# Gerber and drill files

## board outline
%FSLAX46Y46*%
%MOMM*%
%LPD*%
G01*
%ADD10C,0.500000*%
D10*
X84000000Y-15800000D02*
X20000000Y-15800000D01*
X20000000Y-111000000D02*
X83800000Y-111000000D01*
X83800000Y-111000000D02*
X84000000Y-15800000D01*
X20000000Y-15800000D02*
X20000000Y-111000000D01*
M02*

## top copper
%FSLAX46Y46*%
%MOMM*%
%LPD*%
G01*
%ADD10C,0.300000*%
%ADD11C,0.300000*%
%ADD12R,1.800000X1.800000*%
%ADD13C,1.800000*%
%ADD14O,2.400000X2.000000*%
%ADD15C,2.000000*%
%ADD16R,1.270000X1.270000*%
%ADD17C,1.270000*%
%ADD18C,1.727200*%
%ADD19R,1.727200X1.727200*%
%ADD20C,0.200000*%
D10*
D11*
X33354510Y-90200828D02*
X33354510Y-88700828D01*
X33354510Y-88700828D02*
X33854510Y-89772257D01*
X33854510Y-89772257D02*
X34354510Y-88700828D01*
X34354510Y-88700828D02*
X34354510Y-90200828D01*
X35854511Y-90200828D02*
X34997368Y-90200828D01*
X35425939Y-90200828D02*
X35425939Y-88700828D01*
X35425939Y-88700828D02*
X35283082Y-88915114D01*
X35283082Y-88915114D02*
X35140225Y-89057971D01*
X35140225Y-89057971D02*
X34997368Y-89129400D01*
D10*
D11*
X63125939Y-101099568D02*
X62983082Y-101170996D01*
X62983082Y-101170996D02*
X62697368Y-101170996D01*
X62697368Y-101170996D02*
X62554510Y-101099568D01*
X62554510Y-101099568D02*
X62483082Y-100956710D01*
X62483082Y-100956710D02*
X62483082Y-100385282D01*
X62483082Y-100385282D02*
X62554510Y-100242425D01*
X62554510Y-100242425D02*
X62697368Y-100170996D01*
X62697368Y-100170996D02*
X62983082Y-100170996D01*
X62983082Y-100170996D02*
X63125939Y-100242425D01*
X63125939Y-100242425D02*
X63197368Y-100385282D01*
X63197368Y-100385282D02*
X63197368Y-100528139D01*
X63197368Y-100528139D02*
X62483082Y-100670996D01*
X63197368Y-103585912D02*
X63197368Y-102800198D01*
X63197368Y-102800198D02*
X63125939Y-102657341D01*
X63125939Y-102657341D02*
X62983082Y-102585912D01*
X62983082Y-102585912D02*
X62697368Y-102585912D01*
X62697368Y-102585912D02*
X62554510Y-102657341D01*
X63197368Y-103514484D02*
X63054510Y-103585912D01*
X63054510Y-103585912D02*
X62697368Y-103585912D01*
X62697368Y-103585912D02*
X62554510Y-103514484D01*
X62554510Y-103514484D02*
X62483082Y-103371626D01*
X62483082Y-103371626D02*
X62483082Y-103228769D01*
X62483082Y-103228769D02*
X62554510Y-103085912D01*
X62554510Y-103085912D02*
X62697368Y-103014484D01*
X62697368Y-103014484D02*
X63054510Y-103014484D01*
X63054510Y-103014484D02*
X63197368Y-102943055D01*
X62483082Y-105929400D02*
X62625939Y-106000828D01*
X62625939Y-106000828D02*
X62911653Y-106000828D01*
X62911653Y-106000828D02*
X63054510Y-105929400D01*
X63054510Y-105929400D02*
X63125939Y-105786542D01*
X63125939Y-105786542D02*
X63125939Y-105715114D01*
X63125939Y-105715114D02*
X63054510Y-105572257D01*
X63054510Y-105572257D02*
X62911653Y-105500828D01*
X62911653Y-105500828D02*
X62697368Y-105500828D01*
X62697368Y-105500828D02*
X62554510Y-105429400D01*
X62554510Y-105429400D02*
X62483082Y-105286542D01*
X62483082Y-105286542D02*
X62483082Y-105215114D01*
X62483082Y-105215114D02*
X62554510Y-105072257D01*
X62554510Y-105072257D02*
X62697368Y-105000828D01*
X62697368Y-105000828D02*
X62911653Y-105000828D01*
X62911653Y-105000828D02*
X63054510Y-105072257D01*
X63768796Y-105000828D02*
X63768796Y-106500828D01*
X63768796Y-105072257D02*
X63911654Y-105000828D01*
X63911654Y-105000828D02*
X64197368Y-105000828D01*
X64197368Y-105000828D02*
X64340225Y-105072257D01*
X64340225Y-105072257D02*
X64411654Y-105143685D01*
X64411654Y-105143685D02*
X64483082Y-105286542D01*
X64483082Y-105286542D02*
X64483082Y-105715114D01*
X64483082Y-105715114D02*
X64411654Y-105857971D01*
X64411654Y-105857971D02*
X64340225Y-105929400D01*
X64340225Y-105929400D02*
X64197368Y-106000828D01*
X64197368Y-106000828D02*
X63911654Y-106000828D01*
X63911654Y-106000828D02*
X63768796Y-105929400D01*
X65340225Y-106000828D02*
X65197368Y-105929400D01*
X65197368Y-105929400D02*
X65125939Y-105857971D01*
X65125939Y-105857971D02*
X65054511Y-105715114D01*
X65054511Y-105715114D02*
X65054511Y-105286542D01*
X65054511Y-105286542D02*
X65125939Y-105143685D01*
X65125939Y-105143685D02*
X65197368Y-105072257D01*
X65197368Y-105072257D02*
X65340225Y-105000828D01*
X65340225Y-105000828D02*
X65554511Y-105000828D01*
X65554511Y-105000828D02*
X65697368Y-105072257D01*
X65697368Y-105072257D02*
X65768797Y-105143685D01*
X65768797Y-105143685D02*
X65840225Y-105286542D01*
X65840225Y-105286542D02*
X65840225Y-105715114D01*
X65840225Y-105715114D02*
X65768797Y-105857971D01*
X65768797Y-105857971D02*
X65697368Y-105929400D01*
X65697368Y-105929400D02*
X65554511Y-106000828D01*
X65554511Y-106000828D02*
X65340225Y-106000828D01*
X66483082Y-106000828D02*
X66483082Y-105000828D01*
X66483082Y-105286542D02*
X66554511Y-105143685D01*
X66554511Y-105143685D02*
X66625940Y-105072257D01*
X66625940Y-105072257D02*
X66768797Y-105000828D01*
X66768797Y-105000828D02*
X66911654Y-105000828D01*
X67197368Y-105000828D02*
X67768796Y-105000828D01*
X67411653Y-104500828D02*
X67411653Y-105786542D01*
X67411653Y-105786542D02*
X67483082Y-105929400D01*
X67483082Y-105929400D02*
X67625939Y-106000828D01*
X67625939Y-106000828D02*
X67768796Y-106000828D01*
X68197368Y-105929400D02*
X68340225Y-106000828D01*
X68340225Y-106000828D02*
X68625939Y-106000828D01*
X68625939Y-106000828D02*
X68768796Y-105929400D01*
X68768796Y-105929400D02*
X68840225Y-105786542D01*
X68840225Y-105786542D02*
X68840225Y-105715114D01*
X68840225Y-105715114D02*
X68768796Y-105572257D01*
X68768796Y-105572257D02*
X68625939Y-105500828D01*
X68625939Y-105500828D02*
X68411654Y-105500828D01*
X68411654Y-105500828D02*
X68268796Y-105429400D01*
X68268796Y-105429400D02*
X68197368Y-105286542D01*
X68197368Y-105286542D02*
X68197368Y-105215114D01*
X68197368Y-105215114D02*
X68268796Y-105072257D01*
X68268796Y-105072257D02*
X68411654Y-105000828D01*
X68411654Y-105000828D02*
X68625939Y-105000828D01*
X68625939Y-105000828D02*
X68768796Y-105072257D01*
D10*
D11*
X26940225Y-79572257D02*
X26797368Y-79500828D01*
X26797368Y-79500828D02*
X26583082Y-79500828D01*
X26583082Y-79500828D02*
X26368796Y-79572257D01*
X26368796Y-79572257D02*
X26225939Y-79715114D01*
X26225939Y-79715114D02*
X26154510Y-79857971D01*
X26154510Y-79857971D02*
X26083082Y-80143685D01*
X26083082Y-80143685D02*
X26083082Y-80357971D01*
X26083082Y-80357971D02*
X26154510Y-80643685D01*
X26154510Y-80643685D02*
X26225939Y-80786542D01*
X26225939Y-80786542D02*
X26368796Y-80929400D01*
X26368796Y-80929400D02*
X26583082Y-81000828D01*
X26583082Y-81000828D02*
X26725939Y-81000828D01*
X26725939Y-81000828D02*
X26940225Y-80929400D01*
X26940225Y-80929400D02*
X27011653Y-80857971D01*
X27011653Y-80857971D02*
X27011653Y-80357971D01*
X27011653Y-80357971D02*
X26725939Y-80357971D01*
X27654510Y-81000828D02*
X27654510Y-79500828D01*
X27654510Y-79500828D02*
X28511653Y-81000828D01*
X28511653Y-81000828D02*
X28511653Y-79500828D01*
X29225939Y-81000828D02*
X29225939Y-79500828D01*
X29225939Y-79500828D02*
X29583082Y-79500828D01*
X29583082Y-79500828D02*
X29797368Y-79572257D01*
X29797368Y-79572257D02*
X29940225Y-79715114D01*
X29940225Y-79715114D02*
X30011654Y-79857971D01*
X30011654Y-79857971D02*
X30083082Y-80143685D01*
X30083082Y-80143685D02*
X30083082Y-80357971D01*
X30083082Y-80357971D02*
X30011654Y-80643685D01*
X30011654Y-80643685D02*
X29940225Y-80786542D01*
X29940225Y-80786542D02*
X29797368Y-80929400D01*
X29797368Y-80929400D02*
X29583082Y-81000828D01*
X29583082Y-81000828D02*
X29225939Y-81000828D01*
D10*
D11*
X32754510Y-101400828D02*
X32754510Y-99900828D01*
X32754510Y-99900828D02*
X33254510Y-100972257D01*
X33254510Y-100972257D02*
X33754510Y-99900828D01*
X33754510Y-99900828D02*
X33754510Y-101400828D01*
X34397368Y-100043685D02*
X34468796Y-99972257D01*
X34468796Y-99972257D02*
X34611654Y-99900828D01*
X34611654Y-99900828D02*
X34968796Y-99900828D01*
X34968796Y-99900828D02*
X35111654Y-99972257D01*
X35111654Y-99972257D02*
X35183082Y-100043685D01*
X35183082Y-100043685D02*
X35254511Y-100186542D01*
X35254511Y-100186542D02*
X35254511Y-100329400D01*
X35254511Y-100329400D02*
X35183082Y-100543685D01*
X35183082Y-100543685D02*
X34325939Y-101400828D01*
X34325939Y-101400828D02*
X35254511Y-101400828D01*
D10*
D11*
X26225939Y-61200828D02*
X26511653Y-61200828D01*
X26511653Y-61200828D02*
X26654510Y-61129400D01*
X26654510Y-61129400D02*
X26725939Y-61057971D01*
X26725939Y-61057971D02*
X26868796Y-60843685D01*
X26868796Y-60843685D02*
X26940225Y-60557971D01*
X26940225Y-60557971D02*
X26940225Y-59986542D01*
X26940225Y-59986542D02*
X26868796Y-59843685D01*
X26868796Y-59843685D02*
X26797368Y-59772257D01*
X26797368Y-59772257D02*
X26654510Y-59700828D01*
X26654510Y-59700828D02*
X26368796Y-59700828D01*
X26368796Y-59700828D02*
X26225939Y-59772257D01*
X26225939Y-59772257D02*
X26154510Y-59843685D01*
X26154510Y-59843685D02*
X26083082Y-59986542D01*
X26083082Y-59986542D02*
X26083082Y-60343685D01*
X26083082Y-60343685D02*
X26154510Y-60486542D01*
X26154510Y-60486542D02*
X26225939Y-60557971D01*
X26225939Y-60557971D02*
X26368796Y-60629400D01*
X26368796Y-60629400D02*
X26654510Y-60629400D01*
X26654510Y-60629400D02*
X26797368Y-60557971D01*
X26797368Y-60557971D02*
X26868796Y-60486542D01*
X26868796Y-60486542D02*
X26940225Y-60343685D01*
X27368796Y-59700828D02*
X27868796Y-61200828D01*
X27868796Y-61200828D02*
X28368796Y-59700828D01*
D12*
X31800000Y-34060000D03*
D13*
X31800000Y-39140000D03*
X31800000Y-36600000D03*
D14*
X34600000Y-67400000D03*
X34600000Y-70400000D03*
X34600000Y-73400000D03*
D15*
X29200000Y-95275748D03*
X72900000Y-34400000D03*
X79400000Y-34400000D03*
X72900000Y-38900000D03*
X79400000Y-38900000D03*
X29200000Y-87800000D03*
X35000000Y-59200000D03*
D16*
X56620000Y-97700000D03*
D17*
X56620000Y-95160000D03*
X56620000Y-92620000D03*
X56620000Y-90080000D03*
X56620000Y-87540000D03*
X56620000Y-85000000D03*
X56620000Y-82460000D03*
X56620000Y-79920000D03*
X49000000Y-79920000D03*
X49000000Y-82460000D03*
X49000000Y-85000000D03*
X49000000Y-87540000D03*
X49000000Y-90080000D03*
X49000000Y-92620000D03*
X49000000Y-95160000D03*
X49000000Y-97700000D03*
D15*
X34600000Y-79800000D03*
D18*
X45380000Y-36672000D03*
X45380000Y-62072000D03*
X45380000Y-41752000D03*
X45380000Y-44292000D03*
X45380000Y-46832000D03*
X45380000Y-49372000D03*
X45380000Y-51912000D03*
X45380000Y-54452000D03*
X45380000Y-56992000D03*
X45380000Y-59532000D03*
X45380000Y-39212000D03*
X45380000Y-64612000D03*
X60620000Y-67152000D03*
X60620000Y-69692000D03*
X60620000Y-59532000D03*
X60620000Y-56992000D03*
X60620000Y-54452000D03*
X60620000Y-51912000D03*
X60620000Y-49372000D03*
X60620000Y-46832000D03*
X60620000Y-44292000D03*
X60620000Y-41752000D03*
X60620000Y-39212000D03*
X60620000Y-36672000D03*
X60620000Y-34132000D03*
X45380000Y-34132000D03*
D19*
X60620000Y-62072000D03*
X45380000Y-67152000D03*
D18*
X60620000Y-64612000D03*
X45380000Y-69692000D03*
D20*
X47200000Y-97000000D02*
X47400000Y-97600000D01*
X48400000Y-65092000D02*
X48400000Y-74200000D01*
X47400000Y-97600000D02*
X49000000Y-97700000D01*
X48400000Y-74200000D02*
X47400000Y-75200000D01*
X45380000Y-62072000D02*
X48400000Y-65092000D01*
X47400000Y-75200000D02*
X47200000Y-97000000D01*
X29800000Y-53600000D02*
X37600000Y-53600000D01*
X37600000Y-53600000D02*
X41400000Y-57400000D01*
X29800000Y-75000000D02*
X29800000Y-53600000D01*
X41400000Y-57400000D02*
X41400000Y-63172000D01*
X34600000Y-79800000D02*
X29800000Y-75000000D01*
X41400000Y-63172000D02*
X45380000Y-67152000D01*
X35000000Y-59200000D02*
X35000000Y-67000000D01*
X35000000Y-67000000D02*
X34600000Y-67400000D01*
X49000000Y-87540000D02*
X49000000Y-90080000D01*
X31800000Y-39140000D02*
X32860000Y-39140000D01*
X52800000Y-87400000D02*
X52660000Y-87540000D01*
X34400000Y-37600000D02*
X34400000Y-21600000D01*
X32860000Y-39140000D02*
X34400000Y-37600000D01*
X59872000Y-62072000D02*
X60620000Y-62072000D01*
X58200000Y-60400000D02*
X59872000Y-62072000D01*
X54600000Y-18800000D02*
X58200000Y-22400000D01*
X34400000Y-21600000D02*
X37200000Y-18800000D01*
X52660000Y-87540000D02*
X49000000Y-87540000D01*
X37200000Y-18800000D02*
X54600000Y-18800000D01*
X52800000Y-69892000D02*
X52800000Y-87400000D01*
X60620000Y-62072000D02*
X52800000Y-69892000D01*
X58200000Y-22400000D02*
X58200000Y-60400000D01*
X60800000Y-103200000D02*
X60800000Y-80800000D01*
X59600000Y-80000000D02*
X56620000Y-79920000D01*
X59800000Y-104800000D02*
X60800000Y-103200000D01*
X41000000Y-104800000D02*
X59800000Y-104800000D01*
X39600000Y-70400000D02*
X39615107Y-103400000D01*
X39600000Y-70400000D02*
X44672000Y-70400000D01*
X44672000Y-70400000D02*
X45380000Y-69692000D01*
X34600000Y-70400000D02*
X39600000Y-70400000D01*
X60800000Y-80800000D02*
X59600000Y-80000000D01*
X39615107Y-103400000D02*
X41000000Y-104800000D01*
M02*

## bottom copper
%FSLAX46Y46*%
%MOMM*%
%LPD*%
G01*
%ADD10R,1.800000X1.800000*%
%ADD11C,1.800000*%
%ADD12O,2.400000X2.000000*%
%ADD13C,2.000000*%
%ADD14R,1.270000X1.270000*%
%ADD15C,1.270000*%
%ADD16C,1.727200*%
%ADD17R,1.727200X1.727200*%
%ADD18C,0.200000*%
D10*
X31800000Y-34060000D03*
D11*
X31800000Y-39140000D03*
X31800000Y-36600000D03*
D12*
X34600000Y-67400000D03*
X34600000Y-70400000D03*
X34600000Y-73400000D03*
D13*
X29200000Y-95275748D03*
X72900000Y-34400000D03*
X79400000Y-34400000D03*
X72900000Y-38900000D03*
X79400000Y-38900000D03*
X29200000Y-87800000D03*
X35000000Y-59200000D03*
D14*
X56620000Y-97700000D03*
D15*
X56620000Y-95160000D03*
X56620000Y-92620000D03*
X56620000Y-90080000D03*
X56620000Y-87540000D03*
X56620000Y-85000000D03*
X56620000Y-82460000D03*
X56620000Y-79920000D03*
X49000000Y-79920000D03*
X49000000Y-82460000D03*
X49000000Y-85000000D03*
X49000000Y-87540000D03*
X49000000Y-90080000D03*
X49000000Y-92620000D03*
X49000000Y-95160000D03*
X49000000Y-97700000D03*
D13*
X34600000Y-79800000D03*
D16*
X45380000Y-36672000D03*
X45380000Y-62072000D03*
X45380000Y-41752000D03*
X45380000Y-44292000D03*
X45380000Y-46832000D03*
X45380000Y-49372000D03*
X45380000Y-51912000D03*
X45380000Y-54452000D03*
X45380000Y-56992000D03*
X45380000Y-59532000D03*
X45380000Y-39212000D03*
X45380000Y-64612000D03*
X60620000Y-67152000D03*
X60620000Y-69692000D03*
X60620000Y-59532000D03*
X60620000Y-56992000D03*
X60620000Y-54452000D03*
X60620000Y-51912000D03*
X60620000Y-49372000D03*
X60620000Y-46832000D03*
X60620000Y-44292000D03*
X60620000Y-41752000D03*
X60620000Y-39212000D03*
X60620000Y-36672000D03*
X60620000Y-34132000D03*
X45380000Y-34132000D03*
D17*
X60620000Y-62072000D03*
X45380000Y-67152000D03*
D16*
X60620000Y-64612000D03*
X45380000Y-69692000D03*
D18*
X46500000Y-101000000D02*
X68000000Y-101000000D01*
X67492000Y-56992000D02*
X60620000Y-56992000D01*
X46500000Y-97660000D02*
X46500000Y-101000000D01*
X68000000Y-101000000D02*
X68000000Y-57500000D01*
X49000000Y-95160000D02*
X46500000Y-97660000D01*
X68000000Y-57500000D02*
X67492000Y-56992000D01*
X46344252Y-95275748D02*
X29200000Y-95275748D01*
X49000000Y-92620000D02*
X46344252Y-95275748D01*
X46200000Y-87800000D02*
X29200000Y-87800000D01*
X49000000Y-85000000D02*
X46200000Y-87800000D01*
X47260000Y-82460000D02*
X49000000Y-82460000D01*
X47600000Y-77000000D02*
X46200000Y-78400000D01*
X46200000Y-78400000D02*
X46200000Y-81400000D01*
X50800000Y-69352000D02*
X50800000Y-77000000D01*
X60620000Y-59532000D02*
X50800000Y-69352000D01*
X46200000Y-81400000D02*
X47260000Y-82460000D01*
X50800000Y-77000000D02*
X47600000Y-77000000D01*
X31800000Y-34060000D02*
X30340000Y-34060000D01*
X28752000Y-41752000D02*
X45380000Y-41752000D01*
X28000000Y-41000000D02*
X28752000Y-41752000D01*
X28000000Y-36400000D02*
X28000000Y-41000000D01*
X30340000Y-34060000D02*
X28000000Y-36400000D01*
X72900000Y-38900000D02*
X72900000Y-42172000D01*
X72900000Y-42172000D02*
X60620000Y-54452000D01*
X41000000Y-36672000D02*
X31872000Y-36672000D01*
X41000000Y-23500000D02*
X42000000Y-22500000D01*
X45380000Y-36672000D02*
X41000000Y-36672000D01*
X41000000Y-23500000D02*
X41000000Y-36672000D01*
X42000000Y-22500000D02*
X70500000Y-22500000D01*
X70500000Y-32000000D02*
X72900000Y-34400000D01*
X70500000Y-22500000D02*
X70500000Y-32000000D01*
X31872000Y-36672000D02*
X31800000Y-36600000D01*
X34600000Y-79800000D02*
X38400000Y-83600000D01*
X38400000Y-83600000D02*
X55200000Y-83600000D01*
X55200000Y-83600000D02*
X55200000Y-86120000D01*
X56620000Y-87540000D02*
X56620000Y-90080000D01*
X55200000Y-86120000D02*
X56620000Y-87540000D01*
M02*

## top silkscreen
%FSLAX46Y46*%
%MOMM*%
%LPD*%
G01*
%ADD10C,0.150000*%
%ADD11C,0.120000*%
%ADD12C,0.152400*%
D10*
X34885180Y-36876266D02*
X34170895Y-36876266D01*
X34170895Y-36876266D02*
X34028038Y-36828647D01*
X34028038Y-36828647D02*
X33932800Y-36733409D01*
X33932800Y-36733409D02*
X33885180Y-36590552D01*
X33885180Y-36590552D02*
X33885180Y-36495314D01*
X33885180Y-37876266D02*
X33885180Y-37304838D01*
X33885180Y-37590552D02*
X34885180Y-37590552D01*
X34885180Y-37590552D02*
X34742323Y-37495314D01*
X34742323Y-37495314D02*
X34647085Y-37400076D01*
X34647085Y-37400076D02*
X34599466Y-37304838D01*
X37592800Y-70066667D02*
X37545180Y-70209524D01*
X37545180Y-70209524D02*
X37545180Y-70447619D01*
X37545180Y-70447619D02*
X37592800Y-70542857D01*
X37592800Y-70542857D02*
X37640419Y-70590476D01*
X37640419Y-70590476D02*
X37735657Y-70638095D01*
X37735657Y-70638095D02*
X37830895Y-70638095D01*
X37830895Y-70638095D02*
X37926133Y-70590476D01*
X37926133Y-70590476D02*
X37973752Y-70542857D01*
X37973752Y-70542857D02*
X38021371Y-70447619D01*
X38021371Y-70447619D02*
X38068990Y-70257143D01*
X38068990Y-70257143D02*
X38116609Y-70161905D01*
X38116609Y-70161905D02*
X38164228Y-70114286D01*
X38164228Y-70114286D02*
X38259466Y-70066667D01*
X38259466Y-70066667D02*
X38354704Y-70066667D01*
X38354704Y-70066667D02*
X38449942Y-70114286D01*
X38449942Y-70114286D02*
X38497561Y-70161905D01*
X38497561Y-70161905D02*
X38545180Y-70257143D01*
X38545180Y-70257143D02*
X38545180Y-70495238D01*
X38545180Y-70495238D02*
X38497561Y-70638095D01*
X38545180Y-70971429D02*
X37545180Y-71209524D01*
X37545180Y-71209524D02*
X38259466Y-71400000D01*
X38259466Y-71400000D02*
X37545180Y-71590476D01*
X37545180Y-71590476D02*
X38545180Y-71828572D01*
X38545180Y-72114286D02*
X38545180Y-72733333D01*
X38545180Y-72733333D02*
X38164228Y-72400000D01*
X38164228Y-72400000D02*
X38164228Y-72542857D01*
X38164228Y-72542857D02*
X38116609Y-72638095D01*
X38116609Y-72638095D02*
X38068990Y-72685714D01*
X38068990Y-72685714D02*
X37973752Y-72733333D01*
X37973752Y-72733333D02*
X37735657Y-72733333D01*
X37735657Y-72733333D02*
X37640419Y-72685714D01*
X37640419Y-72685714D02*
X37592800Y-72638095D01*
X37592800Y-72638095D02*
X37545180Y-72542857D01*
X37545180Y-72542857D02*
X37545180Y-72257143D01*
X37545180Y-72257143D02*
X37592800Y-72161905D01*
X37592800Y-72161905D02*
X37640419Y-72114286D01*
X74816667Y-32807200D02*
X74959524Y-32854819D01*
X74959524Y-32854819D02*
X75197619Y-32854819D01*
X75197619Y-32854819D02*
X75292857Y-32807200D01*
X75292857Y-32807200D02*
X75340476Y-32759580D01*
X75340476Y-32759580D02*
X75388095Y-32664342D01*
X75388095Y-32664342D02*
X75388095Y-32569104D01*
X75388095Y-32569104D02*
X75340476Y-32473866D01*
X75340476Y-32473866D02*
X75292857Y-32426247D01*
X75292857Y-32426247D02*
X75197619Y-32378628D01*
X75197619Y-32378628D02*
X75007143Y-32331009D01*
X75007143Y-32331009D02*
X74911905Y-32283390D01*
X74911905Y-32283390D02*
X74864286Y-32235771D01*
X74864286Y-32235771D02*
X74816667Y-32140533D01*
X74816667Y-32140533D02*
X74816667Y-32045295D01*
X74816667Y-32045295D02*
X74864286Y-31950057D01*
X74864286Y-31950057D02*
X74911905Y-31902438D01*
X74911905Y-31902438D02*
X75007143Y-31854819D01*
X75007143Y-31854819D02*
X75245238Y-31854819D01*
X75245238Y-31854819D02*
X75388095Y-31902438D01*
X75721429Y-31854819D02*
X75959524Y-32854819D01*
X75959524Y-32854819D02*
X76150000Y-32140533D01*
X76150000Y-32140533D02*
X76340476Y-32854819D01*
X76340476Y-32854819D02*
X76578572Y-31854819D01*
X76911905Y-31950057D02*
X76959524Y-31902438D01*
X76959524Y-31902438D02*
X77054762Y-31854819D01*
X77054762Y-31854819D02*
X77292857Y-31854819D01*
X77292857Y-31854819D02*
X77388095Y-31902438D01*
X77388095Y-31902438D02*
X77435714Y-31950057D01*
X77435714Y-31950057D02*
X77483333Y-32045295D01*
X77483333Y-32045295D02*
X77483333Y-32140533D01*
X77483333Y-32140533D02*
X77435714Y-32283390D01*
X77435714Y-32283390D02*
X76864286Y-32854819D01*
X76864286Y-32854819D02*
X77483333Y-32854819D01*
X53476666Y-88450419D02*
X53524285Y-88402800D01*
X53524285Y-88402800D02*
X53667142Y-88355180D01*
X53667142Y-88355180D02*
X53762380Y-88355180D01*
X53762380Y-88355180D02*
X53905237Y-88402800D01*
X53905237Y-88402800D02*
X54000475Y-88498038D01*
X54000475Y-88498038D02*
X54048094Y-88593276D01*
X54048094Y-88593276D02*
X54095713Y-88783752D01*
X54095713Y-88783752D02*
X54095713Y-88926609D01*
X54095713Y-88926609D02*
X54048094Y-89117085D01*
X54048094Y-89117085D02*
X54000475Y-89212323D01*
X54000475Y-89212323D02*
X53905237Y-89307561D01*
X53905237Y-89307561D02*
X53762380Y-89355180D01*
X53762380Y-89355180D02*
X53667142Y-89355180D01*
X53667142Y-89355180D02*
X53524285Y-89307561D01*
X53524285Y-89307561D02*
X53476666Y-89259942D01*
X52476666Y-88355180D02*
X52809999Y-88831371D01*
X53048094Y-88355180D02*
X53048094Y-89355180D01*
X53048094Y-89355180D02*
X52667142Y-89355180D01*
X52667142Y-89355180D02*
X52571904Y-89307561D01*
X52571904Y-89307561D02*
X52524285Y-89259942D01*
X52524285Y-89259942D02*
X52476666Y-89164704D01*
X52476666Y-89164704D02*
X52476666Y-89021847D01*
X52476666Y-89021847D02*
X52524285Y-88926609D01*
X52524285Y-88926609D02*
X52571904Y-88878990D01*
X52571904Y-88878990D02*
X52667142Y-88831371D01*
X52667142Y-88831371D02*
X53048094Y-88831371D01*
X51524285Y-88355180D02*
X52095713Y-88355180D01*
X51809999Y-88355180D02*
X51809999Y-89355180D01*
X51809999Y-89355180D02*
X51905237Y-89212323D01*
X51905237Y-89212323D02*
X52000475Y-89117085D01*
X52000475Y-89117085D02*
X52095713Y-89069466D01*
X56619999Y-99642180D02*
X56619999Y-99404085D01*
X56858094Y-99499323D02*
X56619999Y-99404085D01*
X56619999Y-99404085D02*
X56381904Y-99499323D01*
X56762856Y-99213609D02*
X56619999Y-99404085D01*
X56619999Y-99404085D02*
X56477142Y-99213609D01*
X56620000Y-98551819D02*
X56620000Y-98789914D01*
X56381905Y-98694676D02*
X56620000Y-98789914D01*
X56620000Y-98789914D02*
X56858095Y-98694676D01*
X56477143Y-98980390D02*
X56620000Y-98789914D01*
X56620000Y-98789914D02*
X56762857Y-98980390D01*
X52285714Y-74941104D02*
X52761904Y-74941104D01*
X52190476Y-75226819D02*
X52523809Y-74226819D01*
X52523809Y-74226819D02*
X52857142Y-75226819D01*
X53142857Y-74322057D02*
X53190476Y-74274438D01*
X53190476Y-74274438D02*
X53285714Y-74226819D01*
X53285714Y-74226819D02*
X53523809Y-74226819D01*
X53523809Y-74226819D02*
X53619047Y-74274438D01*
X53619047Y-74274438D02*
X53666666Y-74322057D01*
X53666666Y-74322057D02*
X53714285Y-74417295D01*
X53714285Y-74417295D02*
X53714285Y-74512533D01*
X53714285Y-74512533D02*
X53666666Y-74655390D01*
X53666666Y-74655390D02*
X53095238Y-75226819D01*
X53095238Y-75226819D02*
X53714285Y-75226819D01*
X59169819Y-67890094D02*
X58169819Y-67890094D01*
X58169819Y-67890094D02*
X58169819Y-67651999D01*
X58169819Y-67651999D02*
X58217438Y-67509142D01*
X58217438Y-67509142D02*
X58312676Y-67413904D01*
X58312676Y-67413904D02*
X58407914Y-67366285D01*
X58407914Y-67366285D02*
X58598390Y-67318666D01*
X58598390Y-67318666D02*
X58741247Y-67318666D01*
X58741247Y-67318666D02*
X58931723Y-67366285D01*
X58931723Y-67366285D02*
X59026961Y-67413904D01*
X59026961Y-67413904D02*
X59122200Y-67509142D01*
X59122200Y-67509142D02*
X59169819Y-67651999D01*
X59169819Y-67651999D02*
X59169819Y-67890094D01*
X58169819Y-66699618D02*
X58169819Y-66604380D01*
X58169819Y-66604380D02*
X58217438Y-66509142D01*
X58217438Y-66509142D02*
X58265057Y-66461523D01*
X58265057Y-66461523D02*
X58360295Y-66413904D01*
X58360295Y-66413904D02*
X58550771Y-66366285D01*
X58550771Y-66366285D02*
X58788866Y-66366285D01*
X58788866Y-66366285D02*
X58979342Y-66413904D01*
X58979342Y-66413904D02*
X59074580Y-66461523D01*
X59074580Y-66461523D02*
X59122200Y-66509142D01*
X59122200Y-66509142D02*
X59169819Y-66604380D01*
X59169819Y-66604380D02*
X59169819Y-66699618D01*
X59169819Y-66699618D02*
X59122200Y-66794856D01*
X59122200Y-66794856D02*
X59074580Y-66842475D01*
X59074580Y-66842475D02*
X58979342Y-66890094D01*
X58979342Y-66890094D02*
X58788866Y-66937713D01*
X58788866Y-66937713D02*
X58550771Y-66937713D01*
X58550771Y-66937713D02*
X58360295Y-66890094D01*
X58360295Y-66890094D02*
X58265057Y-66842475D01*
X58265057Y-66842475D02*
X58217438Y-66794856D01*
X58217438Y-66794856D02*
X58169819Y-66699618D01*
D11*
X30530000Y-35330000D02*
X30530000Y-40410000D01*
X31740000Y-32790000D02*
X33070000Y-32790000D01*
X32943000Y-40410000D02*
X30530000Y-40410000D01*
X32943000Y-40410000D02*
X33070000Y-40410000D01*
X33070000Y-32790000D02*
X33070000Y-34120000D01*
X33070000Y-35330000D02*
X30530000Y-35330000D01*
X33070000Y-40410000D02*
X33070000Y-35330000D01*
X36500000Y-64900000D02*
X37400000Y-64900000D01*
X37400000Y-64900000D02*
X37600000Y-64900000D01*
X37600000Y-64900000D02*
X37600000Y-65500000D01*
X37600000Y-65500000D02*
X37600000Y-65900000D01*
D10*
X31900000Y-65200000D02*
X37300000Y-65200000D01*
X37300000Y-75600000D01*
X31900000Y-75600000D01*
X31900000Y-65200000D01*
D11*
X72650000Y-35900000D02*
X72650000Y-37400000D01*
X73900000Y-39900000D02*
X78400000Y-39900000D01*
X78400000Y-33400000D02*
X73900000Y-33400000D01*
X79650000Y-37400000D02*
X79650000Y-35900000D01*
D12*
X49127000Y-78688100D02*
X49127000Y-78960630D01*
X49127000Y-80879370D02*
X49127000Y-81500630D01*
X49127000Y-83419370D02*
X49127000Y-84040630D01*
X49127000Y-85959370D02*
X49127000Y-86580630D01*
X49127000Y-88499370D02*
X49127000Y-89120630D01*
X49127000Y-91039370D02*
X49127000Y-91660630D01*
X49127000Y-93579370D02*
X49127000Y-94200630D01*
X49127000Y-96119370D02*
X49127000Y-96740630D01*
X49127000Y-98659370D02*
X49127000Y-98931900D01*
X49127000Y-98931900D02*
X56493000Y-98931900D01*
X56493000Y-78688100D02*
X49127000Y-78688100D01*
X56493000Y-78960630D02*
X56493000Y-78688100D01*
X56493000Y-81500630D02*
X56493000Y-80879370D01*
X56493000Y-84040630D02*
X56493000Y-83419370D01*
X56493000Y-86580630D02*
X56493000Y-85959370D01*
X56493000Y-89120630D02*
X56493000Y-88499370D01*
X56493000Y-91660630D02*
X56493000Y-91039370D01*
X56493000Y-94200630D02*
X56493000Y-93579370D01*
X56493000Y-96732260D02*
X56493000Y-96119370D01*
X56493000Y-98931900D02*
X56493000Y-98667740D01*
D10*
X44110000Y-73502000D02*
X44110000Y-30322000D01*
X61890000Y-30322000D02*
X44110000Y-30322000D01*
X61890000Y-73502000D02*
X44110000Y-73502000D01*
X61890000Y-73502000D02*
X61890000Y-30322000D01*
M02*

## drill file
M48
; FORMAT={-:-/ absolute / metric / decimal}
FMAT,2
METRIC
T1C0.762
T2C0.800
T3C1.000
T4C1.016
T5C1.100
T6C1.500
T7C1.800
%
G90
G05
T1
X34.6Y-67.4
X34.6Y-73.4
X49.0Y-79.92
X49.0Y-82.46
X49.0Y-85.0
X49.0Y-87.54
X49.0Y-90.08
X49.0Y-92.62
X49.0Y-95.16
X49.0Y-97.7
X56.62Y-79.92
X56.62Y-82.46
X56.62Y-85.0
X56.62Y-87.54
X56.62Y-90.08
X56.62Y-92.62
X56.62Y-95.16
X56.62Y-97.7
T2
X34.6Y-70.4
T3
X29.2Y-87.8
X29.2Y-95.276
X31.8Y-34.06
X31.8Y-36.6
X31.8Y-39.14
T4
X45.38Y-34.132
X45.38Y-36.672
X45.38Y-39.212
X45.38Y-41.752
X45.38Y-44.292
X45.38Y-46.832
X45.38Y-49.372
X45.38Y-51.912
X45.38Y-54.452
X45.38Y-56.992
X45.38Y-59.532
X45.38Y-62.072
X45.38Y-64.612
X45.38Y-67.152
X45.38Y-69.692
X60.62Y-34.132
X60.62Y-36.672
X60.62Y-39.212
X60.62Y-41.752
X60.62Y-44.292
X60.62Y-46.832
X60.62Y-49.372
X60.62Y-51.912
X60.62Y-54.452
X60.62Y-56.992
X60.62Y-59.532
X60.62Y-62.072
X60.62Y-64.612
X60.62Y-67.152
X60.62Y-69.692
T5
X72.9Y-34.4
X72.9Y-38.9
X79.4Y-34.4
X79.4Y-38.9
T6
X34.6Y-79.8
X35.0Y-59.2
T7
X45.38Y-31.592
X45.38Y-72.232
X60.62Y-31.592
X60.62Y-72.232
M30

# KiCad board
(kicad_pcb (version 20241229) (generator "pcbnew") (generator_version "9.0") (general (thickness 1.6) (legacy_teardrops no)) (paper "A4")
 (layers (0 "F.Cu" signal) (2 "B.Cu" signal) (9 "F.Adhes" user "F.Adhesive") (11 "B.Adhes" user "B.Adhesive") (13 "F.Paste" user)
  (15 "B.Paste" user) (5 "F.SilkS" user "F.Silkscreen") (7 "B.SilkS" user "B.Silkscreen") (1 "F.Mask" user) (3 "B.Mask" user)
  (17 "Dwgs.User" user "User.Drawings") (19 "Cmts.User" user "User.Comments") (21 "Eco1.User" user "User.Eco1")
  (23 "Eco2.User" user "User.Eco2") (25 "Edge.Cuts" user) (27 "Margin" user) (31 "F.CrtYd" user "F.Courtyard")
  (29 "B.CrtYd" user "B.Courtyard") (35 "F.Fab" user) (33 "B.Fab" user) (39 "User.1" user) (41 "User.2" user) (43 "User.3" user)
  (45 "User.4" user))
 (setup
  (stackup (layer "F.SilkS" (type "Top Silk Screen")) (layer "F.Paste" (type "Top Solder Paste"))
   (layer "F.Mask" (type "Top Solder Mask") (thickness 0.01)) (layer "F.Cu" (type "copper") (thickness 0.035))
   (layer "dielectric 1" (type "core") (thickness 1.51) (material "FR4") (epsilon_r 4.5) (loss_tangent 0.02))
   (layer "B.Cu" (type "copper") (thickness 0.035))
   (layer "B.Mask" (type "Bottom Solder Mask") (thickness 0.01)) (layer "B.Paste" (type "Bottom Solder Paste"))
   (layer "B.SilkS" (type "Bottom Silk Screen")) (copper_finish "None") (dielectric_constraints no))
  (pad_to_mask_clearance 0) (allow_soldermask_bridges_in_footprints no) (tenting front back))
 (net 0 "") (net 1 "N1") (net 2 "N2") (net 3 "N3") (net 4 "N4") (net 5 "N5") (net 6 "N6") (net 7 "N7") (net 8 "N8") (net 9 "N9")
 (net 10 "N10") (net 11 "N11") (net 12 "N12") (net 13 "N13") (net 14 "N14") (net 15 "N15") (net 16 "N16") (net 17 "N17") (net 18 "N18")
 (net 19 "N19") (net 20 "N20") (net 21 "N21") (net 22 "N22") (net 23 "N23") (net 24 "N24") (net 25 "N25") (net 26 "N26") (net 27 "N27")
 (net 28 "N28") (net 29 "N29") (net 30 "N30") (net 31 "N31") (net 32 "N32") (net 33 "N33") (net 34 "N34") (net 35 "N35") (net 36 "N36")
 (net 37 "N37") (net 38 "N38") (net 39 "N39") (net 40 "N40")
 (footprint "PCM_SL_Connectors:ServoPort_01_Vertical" (layer "F.Cu") (at 31.8 34.06 -90)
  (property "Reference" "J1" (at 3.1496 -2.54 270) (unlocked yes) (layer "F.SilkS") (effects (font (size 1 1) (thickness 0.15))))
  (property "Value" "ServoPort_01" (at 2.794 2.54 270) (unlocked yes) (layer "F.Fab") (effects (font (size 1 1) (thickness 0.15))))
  (fp_line (start 1.27 1.27) (end 6.35 1.27) (stroke (width 0.12) (type solid)) (layer "F.SilkS"))
  (fp_line (start -1.27 0.06) (end -1.27 -1.27) (stroke (width 0.12) (type solid)) (layer "F.SilkS"))
  (fp_line (start 6.35 -1.143) (end 6.35 1.27) (stroke (width 0.12) (type solid)) (layer "F.SilkS"))
  (fp_line (start 6.35 -1.143) (end 6.35 -1.27) (stroke (width 0.12) (type solid)) (layer "F.SilkS"))
  (fp_line (start -1.27 -1.27) (end 0.06 -1.27) (stroke (width 0.12) (type solid)) (layer "F.SilkS"))
  (fp_line (start 1.27 -1.27) (end 1.27 1.27) (stroke (width 0.12) (type solid)) (layer "F.SilkS"))
  (fp_line (start 6.35 -1.27) (end 1.27 -1.27) (stroke (width 0.12) (type solid)) (layer "F.SilkS"))
  (pad "1" thru_hole rect (at 0 0 270) (size 1.8 1.8) (drill 1) (layers "*.Cu" "*.Mask") (remove_unused_layers no) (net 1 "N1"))
  (pad "GND" thru_hole circle (at 5.08 0 270) (size 1.8 1.8) (drill 1) (layers "*.Cu" "*.Mask") (remove_unused_layers no) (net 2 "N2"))
  (pad "VCC" thru_hole circle (at 2.54 0 270) (size 1.8 1.8) (drill 1) (layers "*.Cu" "*.Mask") (remove_unused_layers no) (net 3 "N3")))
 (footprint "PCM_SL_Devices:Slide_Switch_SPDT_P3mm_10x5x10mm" (layer "F.Cu") (at 34.6 67.4 -90)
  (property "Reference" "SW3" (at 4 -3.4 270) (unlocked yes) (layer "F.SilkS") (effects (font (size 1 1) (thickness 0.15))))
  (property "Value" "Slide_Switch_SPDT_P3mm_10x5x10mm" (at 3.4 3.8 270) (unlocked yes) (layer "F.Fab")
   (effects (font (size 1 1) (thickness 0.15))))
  (fp_line (start -2.5 -1.9) (end -2.5 -2.8) (stroke (width 0.12) (type solid)) (layer "F.SilkS"))
  (fp_line (start -2.5 -2.8) (end -2.5 -3) (stroke (width 0.12) (type solid)) (layer "F.SilkS"))
  (fp_line (start -2.5 -3) (end -1.9 -3) (stroke (width 0.12) (type solid)) (layer "F.SilkS"))
  (fp_line (start -1.9 -3) (end -1.5 -3) (stroke (width 0.12) (type solid)) (layer "F.SilkS"))
  (fp_rect (start -2.2 -2.7) (end 8.2 2.7) (stroke (width 0.15) (type solid)) (fill no) (layer "F.SilkS"))
  (pad "1" thru_hole oval (at 0 0 270) (size 2 2.4) (drill 0.762) (layers "*.Cu" "*.Mask") (remove_unused_layers no) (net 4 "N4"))
  (pad "2" thru_hole oval (at 3 0 270) (size 2 2.4) (drill 0.8) (layers "*.Cu" "*.Mask") (remove_unused_layers no) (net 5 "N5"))
  (pad "3" thru_hole oval (at 6 0 270) (size 2 2.4) (drill 0.762) (layers "*.Cu" "*.Mask") (remove_unused_layers no) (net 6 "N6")))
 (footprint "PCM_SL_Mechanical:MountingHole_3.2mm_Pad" (layer "F.Cu") (at 29.2 95.275748)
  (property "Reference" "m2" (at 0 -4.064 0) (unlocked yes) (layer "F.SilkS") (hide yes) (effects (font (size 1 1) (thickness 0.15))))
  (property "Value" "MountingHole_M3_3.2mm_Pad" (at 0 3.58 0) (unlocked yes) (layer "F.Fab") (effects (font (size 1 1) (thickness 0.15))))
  (pad "1" thru_hole circle (at 0 0) (size 2 2) (drill 1) (layers "*.Cu" "*.Mask") (remove_unused_layers no) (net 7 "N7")))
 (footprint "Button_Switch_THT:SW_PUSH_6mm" (layer "F.Cu") (at 72.9 34.4)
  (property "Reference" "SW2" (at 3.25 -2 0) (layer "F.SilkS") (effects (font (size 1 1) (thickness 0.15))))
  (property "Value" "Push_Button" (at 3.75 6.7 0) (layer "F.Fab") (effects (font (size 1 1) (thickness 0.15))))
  (fp_line (start -0.25 1.5) (end -0.25 3) (stroke (width 0.12) (type solid)) (layer "F.SilkS"))
  (fp_line (start 1 5.5) (end 5.5 5.5) (stroke (width 0.12) (type solid)) (layer "F.SilkS"))
  (fp_line (start 5.5 -1) (end 1 -1) (stroke (width 0.12) (type solid)) (layer "F.SilkS"))
  (fp_line (start 6.75 3) (end 6.75 1.5) (stroke (width 0.12) (type solid)) (layer "F.SilkS"))
  (pad "1" thru_hole circle (at 0 0 90) (size 2 2) (drill 1.1) (layers "*.Cu" "*.Mask") (remove_unused_layers no) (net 3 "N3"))
  (pad "1" thru_hole circle (at 6.5 0 90) (size 2 2) (drill 1.1) (layers "*.Cu" "*.Mask") (remove_unused_layers no) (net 3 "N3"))
  (pad "2" thru_hole circle (at 0 4.5 90) (size 2 2) (drill 1.1) (layers "*.Cu" "*.Mask") (remove_unused_layers no) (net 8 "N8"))
  (pad "2" thru_hole circle (at 6.5 4.5 90) (size 2 2) (drill 1.1) (layers "*.Cu" "*.Mask") (remove_unused_layers no) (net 8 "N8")))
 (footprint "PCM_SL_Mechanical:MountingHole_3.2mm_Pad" (layer "F.Cu") (at 29.2 87.8)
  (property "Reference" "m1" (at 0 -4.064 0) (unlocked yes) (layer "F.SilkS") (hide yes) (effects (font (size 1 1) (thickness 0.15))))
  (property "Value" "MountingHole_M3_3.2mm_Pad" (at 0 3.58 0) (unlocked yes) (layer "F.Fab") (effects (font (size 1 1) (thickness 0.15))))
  (pad "1" thru_hole circle (at 0 0) (size 2 2) (drill 1) (layers "*.Cu" "*.Mask") (remove_unused_layers no) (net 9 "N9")))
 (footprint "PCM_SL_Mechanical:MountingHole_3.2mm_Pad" (layer "F.Cu") (at 35 59.2)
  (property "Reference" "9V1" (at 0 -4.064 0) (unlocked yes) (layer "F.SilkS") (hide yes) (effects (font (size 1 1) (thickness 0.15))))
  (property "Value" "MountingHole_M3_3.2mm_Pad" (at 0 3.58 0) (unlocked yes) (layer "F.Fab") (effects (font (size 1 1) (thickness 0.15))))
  (pad "1" thru_hole circle (at 0 0) (size 2 2) (drill 1.5) (layers "*.Cu" "*.Mask") (remove_unused_layers no) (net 4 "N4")))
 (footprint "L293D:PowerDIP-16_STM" (layer "F.Cu") (at 56.62 97.7 180)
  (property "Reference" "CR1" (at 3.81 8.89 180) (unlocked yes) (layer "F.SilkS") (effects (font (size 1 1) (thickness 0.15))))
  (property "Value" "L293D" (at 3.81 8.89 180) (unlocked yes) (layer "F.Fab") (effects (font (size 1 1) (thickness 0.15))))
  (fp_line (start 7.493 19.0119) (end 7.493 18.73937) (stroke (width 0.1524) (type solid)) (layer "F.SilkS"))
  (fp_line (start 7.493 16.82063) (end 7.493 16.19937) (stroke (width 0.1524) (type solid)) (layer "F.SilkS"))
  (fp_line (start 7.493 14.28063) (end 7.493 13.65937) (stroke (width 0.1524) (type solid)) (layer "F.SilkS"))
  (fp_line (start 7.493 11.74063) (end 7.493 11.11937) (stroke (width 0.1524) (type solid)) (layer "F.SilkS"))
  (fp_line (start 7.493 9.20063) (end 7.493 8.57937) (stroke (width 0.1524) (type solid)) (layer "F.SilkS"))
  (fp_line (start 7.493 6.66063) (end 7.493 6.03937) (stroke (width 0.1524) (type solid)) (layer "F.SilkS"))
  (fp_line (start 7.493 4.12063) (end 7.493 3.49937) (stroke (width 0.1524) (type solid)) (layer "F.SilkS"))
  (fp_line (start 7.493 1.58063) (end 7.493 0.95937) (stroke (width 0.1524) (type solid)) (layer "F.SilkS"))
  (fp_line (start 7.493 -0.95937) (end 7.493 -1.2319) (stroke (width 0.1524) (type solid)) (layer "F.SilkS"))
  (fp_line (start 7.493 -1.2319) (end 0.127 -1.2319) (stroke (width 0.1524) (type solid)) (layer "F.SilkS"))
  (fp_line (start 0.127 19.0119) (end 7.493 19.0119) (stroke (width 0.1524) (type solid)) (layer "F.SilkS"))
  (fp_line (start 0.127 18.73937) (end 0.127 19.0119) (stroke (width 0.1524) (type solid)) (layer "F.SilkS"))
  (fp_line (start 0.127 16.19937) (end 0.127 16.82063) (stroke (width 0.1524) (type solid)) (layer "F.SilkS"))
  (fp_line (start 0.127 13.65937) (end 0.127 14.28063) (stroke (width 0.1524) (type solid)) (layer "F.SilkS"))
  (fp_line (start 0.127 11.11937) (end 0.127 11.74063) (stroke (width 0.1524) (type solid)) (layer "F.SilkS"))
  (fp_line (start 0.127 8.57937) (end 0.127 9.20063) (stroke (width 0.1524) (type solid)) (layer "F.SilkS"))
  (fp_line (start 0.127 6.03937) (end 0.127 6.66063) (stroke (width 0.1524) (type solid)) (layer "F.SilkS"))
  (fp_line (start 0.127 3.49937) (end 0.127 4.12063) (stroke (width 0.1524) (type solid)) (layer "F.SilkS"))
  (fp_line (start 0.127 0.96774) (end 0.127 1.58063) (stroke (width 0.1524) (type solid)) (layer "F.SilkS"))
  (fp_line (start 0.127 -1.2319) (end 0.127 -0.96774) (stroke (width 0.1524) (type solid)) (layer "F.SilkS"))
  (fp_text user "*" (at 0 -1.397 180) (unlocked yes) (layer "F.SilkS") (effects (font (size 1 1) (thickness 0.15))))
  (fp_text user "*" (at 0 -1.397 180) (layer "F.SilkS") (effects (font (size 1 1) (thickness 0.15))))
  (pad "1" thru_hole rect (at 0 0 180) (size 1.27 1.27) (drill 0.762) (layers "*.Cu" "*.Mask") (remove_unused_layers no) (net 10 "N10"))
  (pad "2" thru_hole circle (at 0 2.54 180) (size 1.27 1.27) (drill 0.762) (layers "*.Cu" "*.Mask") (remove_unused_layers no) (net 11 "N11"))
  (pad "3" thru_hole circle (at 0 5.08 180) (size 1.27 1.27) (drill 0.762) (layers "*.Cu" "*.Mask") (remove_unused_layers no) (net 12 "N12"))
  (pad "4" thru_hole circle (at 0 7.62 180) (size 1.27 1.27) (drill 0.762) (layers "*.Cu" "*.Mask") (remove_unused_layers no) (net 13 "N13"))
  (pad "5" thru_hole circle (at 0 10.16 180) (size 1.27 1.27) (drill 0.762) (layers "*.Cu" "*.Mask") (remove_unused_layers no)
   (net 13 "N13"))
  (pad "6" thru_hole circle (at 0 12.7 180) (size 1.27 1.27) (drill 0.762) (layers "*.Cu" "*.Mask") (remove_unused_layers no) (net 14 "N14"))
  (pad "7" thru_hole circle (at 0 15.24 180) (size 1.27 1.27) (drill 0.762) (layers "*.Cu" "*.Mask") (remove_unused_layers no)
   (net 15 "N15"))
  (pad "8" thru_hole circle (at 0 17.78 180) (size 1.27 1.27) (drill 0.762) (layers "*.Cu" "*.Mask") (remove_unused_layers no) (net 5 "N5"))
  (pad "9" thru_hole circle (at 7.62 17.78 180) (size 1.27 1.27) (drill 0.762) (layers "*.Cu" "*.Mask") (remove_unused_layers no)
   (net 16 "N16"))
  (pad "10" thru_hole circle (at 7.62 15.24 180) (size 1.27 1.27) (drill 0.762) (layers "*.Cu" "*.Mask") (remove_unused_layers no)
   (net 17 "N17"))
  (pad "11" thru_hole circle (at 7.62 12.7 180) (size 1.27 1.27) (drill 0.762) (layers "*.Cu" "*.Mask") (remove_unused_layers no)
   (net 9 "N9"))
  (pad "12" thru_hole circle (at 7.62 10.16 180) (size 1.27 1.27) (drill 0.762) (layers "*.Cu" "*.Mask") (remove_unused_layers no)
   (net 2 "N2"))
  (pad "13" thru_hole circle (at 7.62 7.62 180) (size 1.27 1.27) (drill 0.762) (layers "*.Cu" "*.Mask") (remove_unused_layers no)
   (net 2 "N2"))
  (pad "14" thru_hole circle (at 7.62 5.08 180) (size 1.27 1.27) (drill 0.762) (layers "*.Cu" "*.Mask") (remove_unused_layers no)
   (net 7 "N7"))
  (pad "15" thru_hole circle (at 7.62 2.54 180) (size 1.27 1.27) (drill 0.762) (layers "*.Cu" "*.Mask") (remove_unused_layers no)
   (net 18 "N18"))
  (pad "16" thru_hole circle (at 7.62 0 180) (size 1.27 1.27) (drill 0.762) (layers "*.Cu" "*.Mask") (remove_unused_layers no)
   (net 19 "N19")))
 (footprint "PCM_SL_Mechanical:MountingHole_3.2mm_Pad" (layer "F.Cu") (at 34.6 79.8)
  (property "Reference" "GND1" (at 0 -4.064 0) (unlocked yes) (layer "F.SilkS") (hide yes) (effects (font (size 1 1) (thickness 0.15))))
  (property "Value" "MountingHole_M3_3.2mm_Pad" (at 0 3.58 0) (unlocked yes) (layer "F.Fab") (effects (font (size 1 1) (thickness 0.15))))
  (pad "1" thru_hole circle (at 0 0) (size 2 2) (drill 1.5) (layers "*.Cu" "*.Mask") (remove_unused_layers no) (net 13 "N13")))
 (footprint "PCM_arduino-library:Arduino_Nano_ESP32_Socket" (layer "F.Cu") (at 53 30.322 180)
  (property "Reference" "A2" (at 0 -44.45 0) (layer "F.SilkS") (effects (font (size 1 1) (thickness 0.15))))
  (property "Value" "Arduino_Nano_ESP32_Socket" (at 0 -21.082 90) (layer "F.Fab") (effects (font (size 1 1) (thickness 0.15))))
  (fp_line (start 8.89 -43.18) (end 8.89 0) (stroke (width 0.15) (type solid)) (layer "F.SilkS"))
  (fp_line (start -8.89 0) (end 8.89 0) (stroke (width 0.15) (type solid)) (layer "F.SilkS"))
  (fp_line (start -8.89 -43.18) (end 8.89 -43.18) (stroke (width 0.15) (type solid)) (layer "F.SilkS"))
  (fp_line (start -8.89 -43.18) (end -8.89 0) (stroke (width 0.15) (type solid)) (layer "F.SilkS"))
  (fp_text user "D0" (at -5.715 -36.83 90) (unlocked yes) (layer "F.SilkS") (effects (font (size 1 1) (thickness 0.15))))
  (pad "" np_thru_hole circle (at -7.62 -41.91 180) (size 1.8 1.8) (drill 1.8) (layers "*.Cu" "*.Mask"))
  (pad "" np_thru_hole circle (at -7.62 -1.27 180) (size 1.8 1.8) (drill 1.8) (layers "*.Cu" "*.Mask"))
  (pad "" np_thru_hole circle (at 7.62 -41.91 180) (size 1.8 1.8) (drill 1.8) (layers "*.Cu" "*.Mask"))
  (pad "" np_thru_hole circle (at 7.62 -1.27 180) (size 1.8 1.8) (drill 1.8) (layers "*.Cu" "*.Mask"))
  (pad "3V3" thru_hole circle (at 7.62 -6.35 180) (size 1.7272 1.7272) (drill 1.016) (layers "*.Cu" "*.Mask") (remove_unused_layers no)
   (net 3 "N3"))
  (pad "5V" thru_hole circle (at 7.62 -31.75 180) (size 1.7272 1.7272) (drill 1.016) (layers "*.Cu" "*.Mask") (remove_unused_layers no)
   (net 19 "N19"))
  (pad "A0" thru_hole circle (at 7.62 -11.43 180) (size 1.7272 1.7272) (drill 1.016) (layers "*.Cu" "*.Mask") (remove_unused_layers no)
   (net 1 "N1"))
  (pad "A1" thru_hole circle (at 7.62 -13.97 180) (size 1.7272 1.7272) (drill 1.016) (layers "*.Cu" "*.Mask") (remove_unused_layers no)
   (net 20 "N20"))
  (pad "A2" thru_hole circle (at 7.62 -16.51 180) (size 1.7272 1.7272) (drill 1.016) (layers "*.Cu" "*.Mask") (remove_unused_layers no)
   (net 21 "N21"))
  (pad "A3" thru_hole circle (at 7.62 -19.05 180) (size 1.7272 1.7272) (drill 1.016) (layers "*.Cu" "*.Mask") (remove_unused_layers no)
   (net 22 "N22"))
  (pad "A4" thru_hole circle (at 7.62 -21.59 180) (size 1.7272 1.7272) (drill 1.016) (layers "*.Cu" "*.Mask") (remove_unused_layers no)
   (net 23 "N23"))
  (pad "A5" thru_hole circle (at 7.62 -24.13 180) (size 1.7272 1.7272) (drill 1.016) (layers "*.Cu" "*.Mask") (remove_unused_layers no)
   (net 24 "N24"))
  (pad "A6" thru_hole circle (at 7.62 -26.67 180) (size 1.7272 1.7272) (drill 1.016) (layers "*.Cu" "*.Mask") (remove_unused_layers no)
   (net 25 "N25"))
  (pad "A7" thru_hole circle (at 7.62 -29.21 180) (size 1.7272 1.7272) (drill 1.016) (layers "*.Cu" "*.Mask") (remove_unused_layers no)
   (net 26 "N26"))
  (pad "B0" thru_hole circle (at 7.62 -8.89 180) (size 1.7272 1.7272) (drill 1.016) (layers "*.Cu" "*.Mask") (remove_unused_layers no)
   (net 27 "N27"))
  (pad "B1" thru_hole circle (at 7.62 -34.29 180) (size 1.7272 1.7272) (drill 1.016) (layers "*.Cu" "*.Mask") (remove_unused_layers no)
   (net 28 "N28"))
  (pad "D0" thru_hole circle (at -7.62 -36.83 180) (size 1.7272 1.7272) (drill 1.016) (layers "*.Cu" "*.Mask") (remove_unused_layers no)
   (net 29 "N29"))
  (pad "D1" thru_hole circle (at -7.62 -39.37 180) (size 1.7272 1.7272) (drill 1.016) (layers "*.Cu" "*.Mask") (remove_unused_layers no)
   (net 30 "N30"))
  (pad "D2" thru_hole circle (at -7.62 -29.21 180) (size 1.7272 1.7272) (drill 1.016) (layers "*.Cu" "*.Mask") (remove_unused_layers no)
   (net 17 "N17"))
  (pad "D3" thru_hole circle (at -7.62 -26.67 180) (size 1.7272 1.7272) (drill 1.016) (layers "*.Cu" "*.Mask") (remove_unused_layers no)
   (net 18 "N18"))
  (pad "D4" thru_hole circle (at -7.62 -24.13 180) (size 1.7272 1.7272) (drill 1.016) (layers "*.Cu" "*.Mask") (remove_unused_layers no)
   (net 8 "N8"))
  (pad "D5" thru_hole circle (at -7.62 -21.59 180) (size 1.7272 1.7272) (drill 1.016) (layers "*.Cu" "*.Mask") (remove_unused_layers no)
   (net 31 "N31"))
  (pad "D6" thru_hole circle (at -7.62 -19.05 180) (size 1.7272 1.7272) (drill 1.016) (layers "*.Cu" "*.Mask") (remove_unused_layers no)
   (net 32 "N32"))
  (pad "D7" thru_hole circle (at -7.62 -16.51 180) (size 1.7272 1.7272) (drill 1.016) (layers "*.Cu" "*.Mask") (remove_unused_layers no)
   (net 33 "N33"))
  (pad "D8" thru_hole circle (at -7.62 -13.97 180) (size 1.7272 1.7272) (drill 1.016) (layers "*.Cu" "*.Mask") (remove_unused_layers no)
   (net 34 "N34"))
  (pad "D9" thru_hole circle (at -7.62 -11.43 180) (size 1.7272 1.7272) (drill 1.016) (layers "*.Cu" "*.Mask") (remove_unused_layers no)
   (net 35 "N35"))
  (pad "D10" thru_hole circle (at -7.62 -8.89 180) (size 1.7272 1.7272) (drill 1.016) (layers "*.Cu" "*.Mask") (remove_unused_layers no)
   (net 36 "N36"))
  (pad "D11" thru_hole circle (at -7.62 -6.35 180) (size 1.7272 1.7272) (drill 1.016) (layers "*.Cu" "*.Mask") (remove_unused_layers no)
   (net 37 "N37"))
  (pad "D12" thru_hole circle (at -7.62 -3.81 180) (size 1.7272 1.7272) (drill 1.016) (layers "*.Cu" "*.Mask") (remove_unused_layers no)
   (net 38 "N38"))
  (pad "D13" thru_hole circle (at 7.62 -3.81 180) (size 1.7272 1.7272) (drill 1.016) (layers "*.Cu" "*.Mask") (remove_unused_layers no)
   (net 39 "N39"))
  (pad "GND1" thru_hole rect (at -7.62 -31.75 180) (size 1.7272 1.7272) (drill 1.016) (layers "*.Cu" "*.Mask") (remove_unused_layers no)
   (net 2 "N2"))
  (pad "GND2" thru_hole rect (at 7.62 -36.83 180) (size 1.7272 1.7272) (drill 1.016) (layers "*.Cu" "*.Mask") (remove_unused_layers no)
   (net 13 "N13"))
  (pad "RST" thru_hole circle (at -7.62 -34.29 180) (size 1.7272 1.7272) (drill 1.016) (layers "*.Cu" "*.Mask") (remove_unused_layers no)
   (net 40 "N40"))
  (pad "VIN" thru_hole circle (at 7.62 -39.37 180) (size 1.7272 1.7272) (drill 1.016) (layers "*.Cu" "*.Mask") (remove_unused_layers no)
   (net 5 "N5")))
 (gr_line (start 84 15.8) (end 20 15.8) (stroke (width 0.5) (type default)) (layer "Edge.Cuts"))
 (gr_line (start 20 111) (end 83.8 111) (stroke (width 0.5) (type default)) (layer "Edge.Cuts"))
 (gr_line (start 83.8 111) (end 84 15.8) (stroke (width 0.5) (type default)) (layer "Edge.Cuts"))
 (gr_line (start 20 15.8) (end 20 111) (stroke (width 0.5) (type default)) (layer "Edge.Cuts"))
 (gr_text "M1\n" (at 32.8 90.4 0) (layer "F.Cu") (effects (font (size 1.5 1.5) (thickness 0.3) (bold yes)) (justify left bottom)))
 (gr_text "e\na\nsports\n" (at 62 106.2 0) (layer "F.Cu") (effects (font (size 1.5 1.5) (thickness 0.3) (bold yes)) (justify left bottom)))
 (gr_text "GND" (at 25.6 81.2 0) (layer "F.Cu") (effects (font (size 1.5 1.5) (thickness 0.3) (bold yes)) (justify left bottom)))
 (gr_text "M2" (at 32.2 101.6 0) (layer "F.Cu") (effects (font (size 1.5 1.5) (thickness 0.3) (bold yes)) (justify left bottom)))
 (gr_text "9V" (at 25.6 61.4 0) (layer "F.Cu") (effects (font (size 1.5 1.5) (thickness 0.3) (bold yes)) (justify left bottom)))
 (segment (start 46.5 101) (end 68 101) (width 0.2) (layer "B.Cu") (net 18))
 (segment (start 67.492 56.992) (end 60.62 56.992) (width 0.2) (layer "B.Cu") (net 18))
 (segment (start 46.5 97.66) (end 46.5 101) (width 0.2) (layer "B.Cu") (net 18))
 (segment (start 68 101) (end 68 57.5) (width 0.2) (layer "B.Cu") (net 18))
 (segment (start 49 95.16) (end 46.5 97.66) (width 0.2) (layer "B.Cu") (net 18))
 (segment (start 68 57.5) (end 67.492 56.992) (width 0.2) (layer "B.Cu") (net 18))
 (segment (start 46.344252 95.275748) (end 29.2 95.275748) (width 0.2) (layer "B.Cu") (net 7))
 (segment (start 49 92.62) (end 46.344252 95.275748) (width 0.2) (layer "B.Cu") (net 7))
 (segment (start 46.2 87.8) (end 29.2 87.8) (width 0.2) (layer "B.Cu") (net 9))
 (segment (start 49 85) (end 46.2 87.8) (width 0.2) (layer "B.Cu") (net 9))
 (segment (start 47.26 82.46) (end 49 82.46) (width 0.2) (layer "B.Cu") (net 17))
 (segment (start 47.6 77) (end 46.2 78.4) (width 0.2) (layer "B.Cu") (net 17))
 (segment (start 46.2 78.4) (end 46.2 81.4) (width 0.2) (layer "B.Cu") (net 17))
 (segment (start 50.8 69.352) (end 50.8 77) (width 0.2) (layer "B.Cu") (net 17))
 (segment (start 60.62 59.532) (end 50.8 69.352) (width 0.2) (layer "B.Cu") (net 17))
 (segment (start 46.2 81.4) (end 47.26 82.46) (width 0.2) (layer "B.Cu") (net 17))
 (segment (start 50.8 77) (end 47.6 77) (width 0.2) (layer "B.Cu") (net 17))
 (segment (start 31.8 34.06) (end 30.34 34.06) (width 0.2) (layer "B.Cu") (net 1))
 (segment (start 28.752 41.752) (end 45.38 41.752) (width 0.2) (layer "B.Cu") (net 1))
 (segment (start 28 41) (end 28.752 41.752) (width 0.2) (layer "B.Cu") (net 1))
 (segment (start 28 36.4) (end 28 41) (width 0.2) (layer "B.Cu") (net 1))
 (segment (start 30.34 34.06) (end 28 36.4) (width 0.2) (layer "B.Cu") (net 1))
 (segment (start 47.2 97) (end 47.4 97.6) (width 0.2) (layer "F.Cu") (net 19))
 (segment (start 48.4 65.092) (end 48.4 74.2) (width 0.2) (layer "F.Cu") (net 19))
 (segment (start 47.4 97.6) (end 49 97.7) (width 0.2) (layer "F.Cu") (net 19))
 (segment (start 48.4 74.2) (end 47.4 75.2) (width 0.2) (layer "F.Cu") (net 19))
 (segment (start 45.38 62.072) (end 48.4 65.092) (width 0.2) (layer "F.Cu") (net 19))
 (segment (start 47.4 75.2) (end 47.2 97) (width 0.2) (layer "F.Cu") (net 19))
 (segment (start 72.9 38.9) (end 72.9 42.172) (width 0.2) (layer "B.Cu") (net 8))
 (segment (start 72.9 42.172) (end 60.62 54.452) (width 0.2) (layer "B.Cu") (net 8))
 (segment (start 41 36.672) (end 31.872 36.672) (width 0.2) (layer "B.Cu") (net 3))
 (segment (start 41 23.5) (end 42 22.5) (width 0.2) (layer "B.Cu") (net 3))
 (segment (start 45.38 36.672) (end 41 36.672) (width 0.2) (layer "B.Cu") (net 3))
 (segment (start 41 23.5) (end 41 36.672) (width 0.2) (layer "B.Cu") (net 3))
 (segment (start 42 22.5) (end 70.5 22.5) (width 0.2) (layer "B.Cu") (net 3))
 (segment (start 70.5 32) (end 72.9 34.4) (width 0.2) (layer "B.Cu") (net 3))
 (segment (start 70.5 22.5) (end 70.5 32) (width 0.2) (layer "B.Cu") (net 3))
 (segment (start 31.872 36.672) (end 31.8 36.6) (width 0.2) (layer "B.Cu") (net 3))
 (segment (start 29.8 53.6) (end 37.6 53.6) (width 0.2) (layer "F.Cu") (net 13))
 (segment (start 37.6 53.6) (end 41.4 57.4) (width 0.2) (layer "F.Cu") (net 13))
 (segment (start 29.8 75) (end 29.8 53.6) (width 0.2) (layer "F.Cu") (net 13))
 (segment (start 41.4 57.4) (end 41.4 63.172) (width 0.2) (layer "F.Cu") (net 13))
 (segment (start 34.6 79.8) (end 29.8 75) (width 0.2) (layer "F.Cu") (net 13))
 (segment (start 41.4 63.172) (end 45.38 67.152) (width 0.2) (layer "F.Cu") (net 13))
 (segment (start 34.6 79.8) (end 38.4 83.6) (width 0.2) (layer "B.Cu") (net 13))
 (segment (start 38.4 83.6) (end 55.2 83.6) (width 0.2) (layer "B.Cu") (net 13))
 (segment (start 55.2 83.6) (end 55.2 86.12) (width 0.2) (layer "B.Cu") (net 13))
 (segment (start 56.62 87.54) (end 56.62 90.08) (width 0.2) (layer "B.Cu") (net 13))
 (segment (start 55.2 86.12) (end 56.62 87.54) (width 0.2) (layer "B.Cu") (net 13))
 (segment (start 35 59.2) (end 35 67) (width 0.2) (layer "F.Cu") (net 4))
 (segment (start 35 67) (end 34.6 67.4) (width 0.2) (layer "F.Cu") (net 4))
 (segment (start 49 87.54) (end 49 90.08) (width 0.2) (layer "F.Cu") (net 2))
 (segment (start 31.8 39.14) (end 32.86 39.14) (width 0.2) (layer "F.Cu") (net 2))
 (segment (start 52.8 87.4) (end 52.66 87.54) (width 0.2) (layer "F.Cu") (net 2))
 (segment (start 34.4 37.6) (end 34.4 21.6) (width 0.2) (layer "F.Cu") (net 2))
 (segment (start 32.86 39.14) (end 34.4 37.6) (width 0.2) (layer "F.Cu") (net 2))
 (segment (start 59.872 62.072) (end 60.62 62.072) (width 0.2) (layer "F.Cu") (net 2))
 (segment (start 58.2 60.4) (end 59.872 62.072) (width 0.2) (layer "F.Cu") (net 2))
 (segment (start 54.6 18.8) (end 58.2 22.4) (width 0.2) (layer "F.Cu") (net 2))
 (segment (start 34.4 21.6) (end 37.2 18.8) (width 0.2) (layer "F.Cu") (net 2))
 (segment (start 52.66 87.54) (end 49 87.54) (width 0.2) (layer "F.Cu") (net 2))
 (segment (start 37.2 18.8) (end 54.6 18.8) (width 0.2) (layer "F.Cu") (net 2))
 (segment (start 52.8 69.892) (end 52.8 87.4) (width 0.2) (layer "F.Cu") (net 2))
 (segment (start 60.62 62.072) (end 52.8 69.892) (width 0.2) (layer "F.Cu") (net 2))
 (segment (start 58.2 22.4) (end 58.2 60.4) (width 0.2) (layer "F.Cu") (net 2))
 (segment (start 60.8 103.2) (end 60.8 80.8) (width 0.2) (layer "F.Cu") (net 5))
 (segment (start 59.6 80) (end 56.62 79.92) (width 0.2) (layer "F.Cu") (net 5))
 (segment (start 59.8 104.8) (end 60.8 103.2) (width 0.2) (layer "F.Cu") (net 5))
 (segment (start 41 104.8) (end 59.8 104.8) (width 0.2) (layer "F.Cu") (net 5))
 (segment (start 39.6 70.4) (end 39.615107 103.4) (width 0.2) (layer "F.Cu") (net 5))
 (segment (start 39.6 70.4) (end 44.672 70.4) (width 0.2) (layer "F.Cu") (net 5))
 (segment (start 44.672 70.4) (end 45.38 69.692) (width 0.2) (layer "F.Cu") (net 5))
 (segment (start 34.6 70.4) (end 39.6 70.4) (width 0.2) (layer "F.Cu") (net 5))
 (segment (start 60.8 80.8) (end 59.6 80) (width 0.2) (layer "F.Cu") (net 5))
 (segment (start 39.615107 103.4) (end 41 104.8) (width 0.2) (layer "F.Cu") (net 5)))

